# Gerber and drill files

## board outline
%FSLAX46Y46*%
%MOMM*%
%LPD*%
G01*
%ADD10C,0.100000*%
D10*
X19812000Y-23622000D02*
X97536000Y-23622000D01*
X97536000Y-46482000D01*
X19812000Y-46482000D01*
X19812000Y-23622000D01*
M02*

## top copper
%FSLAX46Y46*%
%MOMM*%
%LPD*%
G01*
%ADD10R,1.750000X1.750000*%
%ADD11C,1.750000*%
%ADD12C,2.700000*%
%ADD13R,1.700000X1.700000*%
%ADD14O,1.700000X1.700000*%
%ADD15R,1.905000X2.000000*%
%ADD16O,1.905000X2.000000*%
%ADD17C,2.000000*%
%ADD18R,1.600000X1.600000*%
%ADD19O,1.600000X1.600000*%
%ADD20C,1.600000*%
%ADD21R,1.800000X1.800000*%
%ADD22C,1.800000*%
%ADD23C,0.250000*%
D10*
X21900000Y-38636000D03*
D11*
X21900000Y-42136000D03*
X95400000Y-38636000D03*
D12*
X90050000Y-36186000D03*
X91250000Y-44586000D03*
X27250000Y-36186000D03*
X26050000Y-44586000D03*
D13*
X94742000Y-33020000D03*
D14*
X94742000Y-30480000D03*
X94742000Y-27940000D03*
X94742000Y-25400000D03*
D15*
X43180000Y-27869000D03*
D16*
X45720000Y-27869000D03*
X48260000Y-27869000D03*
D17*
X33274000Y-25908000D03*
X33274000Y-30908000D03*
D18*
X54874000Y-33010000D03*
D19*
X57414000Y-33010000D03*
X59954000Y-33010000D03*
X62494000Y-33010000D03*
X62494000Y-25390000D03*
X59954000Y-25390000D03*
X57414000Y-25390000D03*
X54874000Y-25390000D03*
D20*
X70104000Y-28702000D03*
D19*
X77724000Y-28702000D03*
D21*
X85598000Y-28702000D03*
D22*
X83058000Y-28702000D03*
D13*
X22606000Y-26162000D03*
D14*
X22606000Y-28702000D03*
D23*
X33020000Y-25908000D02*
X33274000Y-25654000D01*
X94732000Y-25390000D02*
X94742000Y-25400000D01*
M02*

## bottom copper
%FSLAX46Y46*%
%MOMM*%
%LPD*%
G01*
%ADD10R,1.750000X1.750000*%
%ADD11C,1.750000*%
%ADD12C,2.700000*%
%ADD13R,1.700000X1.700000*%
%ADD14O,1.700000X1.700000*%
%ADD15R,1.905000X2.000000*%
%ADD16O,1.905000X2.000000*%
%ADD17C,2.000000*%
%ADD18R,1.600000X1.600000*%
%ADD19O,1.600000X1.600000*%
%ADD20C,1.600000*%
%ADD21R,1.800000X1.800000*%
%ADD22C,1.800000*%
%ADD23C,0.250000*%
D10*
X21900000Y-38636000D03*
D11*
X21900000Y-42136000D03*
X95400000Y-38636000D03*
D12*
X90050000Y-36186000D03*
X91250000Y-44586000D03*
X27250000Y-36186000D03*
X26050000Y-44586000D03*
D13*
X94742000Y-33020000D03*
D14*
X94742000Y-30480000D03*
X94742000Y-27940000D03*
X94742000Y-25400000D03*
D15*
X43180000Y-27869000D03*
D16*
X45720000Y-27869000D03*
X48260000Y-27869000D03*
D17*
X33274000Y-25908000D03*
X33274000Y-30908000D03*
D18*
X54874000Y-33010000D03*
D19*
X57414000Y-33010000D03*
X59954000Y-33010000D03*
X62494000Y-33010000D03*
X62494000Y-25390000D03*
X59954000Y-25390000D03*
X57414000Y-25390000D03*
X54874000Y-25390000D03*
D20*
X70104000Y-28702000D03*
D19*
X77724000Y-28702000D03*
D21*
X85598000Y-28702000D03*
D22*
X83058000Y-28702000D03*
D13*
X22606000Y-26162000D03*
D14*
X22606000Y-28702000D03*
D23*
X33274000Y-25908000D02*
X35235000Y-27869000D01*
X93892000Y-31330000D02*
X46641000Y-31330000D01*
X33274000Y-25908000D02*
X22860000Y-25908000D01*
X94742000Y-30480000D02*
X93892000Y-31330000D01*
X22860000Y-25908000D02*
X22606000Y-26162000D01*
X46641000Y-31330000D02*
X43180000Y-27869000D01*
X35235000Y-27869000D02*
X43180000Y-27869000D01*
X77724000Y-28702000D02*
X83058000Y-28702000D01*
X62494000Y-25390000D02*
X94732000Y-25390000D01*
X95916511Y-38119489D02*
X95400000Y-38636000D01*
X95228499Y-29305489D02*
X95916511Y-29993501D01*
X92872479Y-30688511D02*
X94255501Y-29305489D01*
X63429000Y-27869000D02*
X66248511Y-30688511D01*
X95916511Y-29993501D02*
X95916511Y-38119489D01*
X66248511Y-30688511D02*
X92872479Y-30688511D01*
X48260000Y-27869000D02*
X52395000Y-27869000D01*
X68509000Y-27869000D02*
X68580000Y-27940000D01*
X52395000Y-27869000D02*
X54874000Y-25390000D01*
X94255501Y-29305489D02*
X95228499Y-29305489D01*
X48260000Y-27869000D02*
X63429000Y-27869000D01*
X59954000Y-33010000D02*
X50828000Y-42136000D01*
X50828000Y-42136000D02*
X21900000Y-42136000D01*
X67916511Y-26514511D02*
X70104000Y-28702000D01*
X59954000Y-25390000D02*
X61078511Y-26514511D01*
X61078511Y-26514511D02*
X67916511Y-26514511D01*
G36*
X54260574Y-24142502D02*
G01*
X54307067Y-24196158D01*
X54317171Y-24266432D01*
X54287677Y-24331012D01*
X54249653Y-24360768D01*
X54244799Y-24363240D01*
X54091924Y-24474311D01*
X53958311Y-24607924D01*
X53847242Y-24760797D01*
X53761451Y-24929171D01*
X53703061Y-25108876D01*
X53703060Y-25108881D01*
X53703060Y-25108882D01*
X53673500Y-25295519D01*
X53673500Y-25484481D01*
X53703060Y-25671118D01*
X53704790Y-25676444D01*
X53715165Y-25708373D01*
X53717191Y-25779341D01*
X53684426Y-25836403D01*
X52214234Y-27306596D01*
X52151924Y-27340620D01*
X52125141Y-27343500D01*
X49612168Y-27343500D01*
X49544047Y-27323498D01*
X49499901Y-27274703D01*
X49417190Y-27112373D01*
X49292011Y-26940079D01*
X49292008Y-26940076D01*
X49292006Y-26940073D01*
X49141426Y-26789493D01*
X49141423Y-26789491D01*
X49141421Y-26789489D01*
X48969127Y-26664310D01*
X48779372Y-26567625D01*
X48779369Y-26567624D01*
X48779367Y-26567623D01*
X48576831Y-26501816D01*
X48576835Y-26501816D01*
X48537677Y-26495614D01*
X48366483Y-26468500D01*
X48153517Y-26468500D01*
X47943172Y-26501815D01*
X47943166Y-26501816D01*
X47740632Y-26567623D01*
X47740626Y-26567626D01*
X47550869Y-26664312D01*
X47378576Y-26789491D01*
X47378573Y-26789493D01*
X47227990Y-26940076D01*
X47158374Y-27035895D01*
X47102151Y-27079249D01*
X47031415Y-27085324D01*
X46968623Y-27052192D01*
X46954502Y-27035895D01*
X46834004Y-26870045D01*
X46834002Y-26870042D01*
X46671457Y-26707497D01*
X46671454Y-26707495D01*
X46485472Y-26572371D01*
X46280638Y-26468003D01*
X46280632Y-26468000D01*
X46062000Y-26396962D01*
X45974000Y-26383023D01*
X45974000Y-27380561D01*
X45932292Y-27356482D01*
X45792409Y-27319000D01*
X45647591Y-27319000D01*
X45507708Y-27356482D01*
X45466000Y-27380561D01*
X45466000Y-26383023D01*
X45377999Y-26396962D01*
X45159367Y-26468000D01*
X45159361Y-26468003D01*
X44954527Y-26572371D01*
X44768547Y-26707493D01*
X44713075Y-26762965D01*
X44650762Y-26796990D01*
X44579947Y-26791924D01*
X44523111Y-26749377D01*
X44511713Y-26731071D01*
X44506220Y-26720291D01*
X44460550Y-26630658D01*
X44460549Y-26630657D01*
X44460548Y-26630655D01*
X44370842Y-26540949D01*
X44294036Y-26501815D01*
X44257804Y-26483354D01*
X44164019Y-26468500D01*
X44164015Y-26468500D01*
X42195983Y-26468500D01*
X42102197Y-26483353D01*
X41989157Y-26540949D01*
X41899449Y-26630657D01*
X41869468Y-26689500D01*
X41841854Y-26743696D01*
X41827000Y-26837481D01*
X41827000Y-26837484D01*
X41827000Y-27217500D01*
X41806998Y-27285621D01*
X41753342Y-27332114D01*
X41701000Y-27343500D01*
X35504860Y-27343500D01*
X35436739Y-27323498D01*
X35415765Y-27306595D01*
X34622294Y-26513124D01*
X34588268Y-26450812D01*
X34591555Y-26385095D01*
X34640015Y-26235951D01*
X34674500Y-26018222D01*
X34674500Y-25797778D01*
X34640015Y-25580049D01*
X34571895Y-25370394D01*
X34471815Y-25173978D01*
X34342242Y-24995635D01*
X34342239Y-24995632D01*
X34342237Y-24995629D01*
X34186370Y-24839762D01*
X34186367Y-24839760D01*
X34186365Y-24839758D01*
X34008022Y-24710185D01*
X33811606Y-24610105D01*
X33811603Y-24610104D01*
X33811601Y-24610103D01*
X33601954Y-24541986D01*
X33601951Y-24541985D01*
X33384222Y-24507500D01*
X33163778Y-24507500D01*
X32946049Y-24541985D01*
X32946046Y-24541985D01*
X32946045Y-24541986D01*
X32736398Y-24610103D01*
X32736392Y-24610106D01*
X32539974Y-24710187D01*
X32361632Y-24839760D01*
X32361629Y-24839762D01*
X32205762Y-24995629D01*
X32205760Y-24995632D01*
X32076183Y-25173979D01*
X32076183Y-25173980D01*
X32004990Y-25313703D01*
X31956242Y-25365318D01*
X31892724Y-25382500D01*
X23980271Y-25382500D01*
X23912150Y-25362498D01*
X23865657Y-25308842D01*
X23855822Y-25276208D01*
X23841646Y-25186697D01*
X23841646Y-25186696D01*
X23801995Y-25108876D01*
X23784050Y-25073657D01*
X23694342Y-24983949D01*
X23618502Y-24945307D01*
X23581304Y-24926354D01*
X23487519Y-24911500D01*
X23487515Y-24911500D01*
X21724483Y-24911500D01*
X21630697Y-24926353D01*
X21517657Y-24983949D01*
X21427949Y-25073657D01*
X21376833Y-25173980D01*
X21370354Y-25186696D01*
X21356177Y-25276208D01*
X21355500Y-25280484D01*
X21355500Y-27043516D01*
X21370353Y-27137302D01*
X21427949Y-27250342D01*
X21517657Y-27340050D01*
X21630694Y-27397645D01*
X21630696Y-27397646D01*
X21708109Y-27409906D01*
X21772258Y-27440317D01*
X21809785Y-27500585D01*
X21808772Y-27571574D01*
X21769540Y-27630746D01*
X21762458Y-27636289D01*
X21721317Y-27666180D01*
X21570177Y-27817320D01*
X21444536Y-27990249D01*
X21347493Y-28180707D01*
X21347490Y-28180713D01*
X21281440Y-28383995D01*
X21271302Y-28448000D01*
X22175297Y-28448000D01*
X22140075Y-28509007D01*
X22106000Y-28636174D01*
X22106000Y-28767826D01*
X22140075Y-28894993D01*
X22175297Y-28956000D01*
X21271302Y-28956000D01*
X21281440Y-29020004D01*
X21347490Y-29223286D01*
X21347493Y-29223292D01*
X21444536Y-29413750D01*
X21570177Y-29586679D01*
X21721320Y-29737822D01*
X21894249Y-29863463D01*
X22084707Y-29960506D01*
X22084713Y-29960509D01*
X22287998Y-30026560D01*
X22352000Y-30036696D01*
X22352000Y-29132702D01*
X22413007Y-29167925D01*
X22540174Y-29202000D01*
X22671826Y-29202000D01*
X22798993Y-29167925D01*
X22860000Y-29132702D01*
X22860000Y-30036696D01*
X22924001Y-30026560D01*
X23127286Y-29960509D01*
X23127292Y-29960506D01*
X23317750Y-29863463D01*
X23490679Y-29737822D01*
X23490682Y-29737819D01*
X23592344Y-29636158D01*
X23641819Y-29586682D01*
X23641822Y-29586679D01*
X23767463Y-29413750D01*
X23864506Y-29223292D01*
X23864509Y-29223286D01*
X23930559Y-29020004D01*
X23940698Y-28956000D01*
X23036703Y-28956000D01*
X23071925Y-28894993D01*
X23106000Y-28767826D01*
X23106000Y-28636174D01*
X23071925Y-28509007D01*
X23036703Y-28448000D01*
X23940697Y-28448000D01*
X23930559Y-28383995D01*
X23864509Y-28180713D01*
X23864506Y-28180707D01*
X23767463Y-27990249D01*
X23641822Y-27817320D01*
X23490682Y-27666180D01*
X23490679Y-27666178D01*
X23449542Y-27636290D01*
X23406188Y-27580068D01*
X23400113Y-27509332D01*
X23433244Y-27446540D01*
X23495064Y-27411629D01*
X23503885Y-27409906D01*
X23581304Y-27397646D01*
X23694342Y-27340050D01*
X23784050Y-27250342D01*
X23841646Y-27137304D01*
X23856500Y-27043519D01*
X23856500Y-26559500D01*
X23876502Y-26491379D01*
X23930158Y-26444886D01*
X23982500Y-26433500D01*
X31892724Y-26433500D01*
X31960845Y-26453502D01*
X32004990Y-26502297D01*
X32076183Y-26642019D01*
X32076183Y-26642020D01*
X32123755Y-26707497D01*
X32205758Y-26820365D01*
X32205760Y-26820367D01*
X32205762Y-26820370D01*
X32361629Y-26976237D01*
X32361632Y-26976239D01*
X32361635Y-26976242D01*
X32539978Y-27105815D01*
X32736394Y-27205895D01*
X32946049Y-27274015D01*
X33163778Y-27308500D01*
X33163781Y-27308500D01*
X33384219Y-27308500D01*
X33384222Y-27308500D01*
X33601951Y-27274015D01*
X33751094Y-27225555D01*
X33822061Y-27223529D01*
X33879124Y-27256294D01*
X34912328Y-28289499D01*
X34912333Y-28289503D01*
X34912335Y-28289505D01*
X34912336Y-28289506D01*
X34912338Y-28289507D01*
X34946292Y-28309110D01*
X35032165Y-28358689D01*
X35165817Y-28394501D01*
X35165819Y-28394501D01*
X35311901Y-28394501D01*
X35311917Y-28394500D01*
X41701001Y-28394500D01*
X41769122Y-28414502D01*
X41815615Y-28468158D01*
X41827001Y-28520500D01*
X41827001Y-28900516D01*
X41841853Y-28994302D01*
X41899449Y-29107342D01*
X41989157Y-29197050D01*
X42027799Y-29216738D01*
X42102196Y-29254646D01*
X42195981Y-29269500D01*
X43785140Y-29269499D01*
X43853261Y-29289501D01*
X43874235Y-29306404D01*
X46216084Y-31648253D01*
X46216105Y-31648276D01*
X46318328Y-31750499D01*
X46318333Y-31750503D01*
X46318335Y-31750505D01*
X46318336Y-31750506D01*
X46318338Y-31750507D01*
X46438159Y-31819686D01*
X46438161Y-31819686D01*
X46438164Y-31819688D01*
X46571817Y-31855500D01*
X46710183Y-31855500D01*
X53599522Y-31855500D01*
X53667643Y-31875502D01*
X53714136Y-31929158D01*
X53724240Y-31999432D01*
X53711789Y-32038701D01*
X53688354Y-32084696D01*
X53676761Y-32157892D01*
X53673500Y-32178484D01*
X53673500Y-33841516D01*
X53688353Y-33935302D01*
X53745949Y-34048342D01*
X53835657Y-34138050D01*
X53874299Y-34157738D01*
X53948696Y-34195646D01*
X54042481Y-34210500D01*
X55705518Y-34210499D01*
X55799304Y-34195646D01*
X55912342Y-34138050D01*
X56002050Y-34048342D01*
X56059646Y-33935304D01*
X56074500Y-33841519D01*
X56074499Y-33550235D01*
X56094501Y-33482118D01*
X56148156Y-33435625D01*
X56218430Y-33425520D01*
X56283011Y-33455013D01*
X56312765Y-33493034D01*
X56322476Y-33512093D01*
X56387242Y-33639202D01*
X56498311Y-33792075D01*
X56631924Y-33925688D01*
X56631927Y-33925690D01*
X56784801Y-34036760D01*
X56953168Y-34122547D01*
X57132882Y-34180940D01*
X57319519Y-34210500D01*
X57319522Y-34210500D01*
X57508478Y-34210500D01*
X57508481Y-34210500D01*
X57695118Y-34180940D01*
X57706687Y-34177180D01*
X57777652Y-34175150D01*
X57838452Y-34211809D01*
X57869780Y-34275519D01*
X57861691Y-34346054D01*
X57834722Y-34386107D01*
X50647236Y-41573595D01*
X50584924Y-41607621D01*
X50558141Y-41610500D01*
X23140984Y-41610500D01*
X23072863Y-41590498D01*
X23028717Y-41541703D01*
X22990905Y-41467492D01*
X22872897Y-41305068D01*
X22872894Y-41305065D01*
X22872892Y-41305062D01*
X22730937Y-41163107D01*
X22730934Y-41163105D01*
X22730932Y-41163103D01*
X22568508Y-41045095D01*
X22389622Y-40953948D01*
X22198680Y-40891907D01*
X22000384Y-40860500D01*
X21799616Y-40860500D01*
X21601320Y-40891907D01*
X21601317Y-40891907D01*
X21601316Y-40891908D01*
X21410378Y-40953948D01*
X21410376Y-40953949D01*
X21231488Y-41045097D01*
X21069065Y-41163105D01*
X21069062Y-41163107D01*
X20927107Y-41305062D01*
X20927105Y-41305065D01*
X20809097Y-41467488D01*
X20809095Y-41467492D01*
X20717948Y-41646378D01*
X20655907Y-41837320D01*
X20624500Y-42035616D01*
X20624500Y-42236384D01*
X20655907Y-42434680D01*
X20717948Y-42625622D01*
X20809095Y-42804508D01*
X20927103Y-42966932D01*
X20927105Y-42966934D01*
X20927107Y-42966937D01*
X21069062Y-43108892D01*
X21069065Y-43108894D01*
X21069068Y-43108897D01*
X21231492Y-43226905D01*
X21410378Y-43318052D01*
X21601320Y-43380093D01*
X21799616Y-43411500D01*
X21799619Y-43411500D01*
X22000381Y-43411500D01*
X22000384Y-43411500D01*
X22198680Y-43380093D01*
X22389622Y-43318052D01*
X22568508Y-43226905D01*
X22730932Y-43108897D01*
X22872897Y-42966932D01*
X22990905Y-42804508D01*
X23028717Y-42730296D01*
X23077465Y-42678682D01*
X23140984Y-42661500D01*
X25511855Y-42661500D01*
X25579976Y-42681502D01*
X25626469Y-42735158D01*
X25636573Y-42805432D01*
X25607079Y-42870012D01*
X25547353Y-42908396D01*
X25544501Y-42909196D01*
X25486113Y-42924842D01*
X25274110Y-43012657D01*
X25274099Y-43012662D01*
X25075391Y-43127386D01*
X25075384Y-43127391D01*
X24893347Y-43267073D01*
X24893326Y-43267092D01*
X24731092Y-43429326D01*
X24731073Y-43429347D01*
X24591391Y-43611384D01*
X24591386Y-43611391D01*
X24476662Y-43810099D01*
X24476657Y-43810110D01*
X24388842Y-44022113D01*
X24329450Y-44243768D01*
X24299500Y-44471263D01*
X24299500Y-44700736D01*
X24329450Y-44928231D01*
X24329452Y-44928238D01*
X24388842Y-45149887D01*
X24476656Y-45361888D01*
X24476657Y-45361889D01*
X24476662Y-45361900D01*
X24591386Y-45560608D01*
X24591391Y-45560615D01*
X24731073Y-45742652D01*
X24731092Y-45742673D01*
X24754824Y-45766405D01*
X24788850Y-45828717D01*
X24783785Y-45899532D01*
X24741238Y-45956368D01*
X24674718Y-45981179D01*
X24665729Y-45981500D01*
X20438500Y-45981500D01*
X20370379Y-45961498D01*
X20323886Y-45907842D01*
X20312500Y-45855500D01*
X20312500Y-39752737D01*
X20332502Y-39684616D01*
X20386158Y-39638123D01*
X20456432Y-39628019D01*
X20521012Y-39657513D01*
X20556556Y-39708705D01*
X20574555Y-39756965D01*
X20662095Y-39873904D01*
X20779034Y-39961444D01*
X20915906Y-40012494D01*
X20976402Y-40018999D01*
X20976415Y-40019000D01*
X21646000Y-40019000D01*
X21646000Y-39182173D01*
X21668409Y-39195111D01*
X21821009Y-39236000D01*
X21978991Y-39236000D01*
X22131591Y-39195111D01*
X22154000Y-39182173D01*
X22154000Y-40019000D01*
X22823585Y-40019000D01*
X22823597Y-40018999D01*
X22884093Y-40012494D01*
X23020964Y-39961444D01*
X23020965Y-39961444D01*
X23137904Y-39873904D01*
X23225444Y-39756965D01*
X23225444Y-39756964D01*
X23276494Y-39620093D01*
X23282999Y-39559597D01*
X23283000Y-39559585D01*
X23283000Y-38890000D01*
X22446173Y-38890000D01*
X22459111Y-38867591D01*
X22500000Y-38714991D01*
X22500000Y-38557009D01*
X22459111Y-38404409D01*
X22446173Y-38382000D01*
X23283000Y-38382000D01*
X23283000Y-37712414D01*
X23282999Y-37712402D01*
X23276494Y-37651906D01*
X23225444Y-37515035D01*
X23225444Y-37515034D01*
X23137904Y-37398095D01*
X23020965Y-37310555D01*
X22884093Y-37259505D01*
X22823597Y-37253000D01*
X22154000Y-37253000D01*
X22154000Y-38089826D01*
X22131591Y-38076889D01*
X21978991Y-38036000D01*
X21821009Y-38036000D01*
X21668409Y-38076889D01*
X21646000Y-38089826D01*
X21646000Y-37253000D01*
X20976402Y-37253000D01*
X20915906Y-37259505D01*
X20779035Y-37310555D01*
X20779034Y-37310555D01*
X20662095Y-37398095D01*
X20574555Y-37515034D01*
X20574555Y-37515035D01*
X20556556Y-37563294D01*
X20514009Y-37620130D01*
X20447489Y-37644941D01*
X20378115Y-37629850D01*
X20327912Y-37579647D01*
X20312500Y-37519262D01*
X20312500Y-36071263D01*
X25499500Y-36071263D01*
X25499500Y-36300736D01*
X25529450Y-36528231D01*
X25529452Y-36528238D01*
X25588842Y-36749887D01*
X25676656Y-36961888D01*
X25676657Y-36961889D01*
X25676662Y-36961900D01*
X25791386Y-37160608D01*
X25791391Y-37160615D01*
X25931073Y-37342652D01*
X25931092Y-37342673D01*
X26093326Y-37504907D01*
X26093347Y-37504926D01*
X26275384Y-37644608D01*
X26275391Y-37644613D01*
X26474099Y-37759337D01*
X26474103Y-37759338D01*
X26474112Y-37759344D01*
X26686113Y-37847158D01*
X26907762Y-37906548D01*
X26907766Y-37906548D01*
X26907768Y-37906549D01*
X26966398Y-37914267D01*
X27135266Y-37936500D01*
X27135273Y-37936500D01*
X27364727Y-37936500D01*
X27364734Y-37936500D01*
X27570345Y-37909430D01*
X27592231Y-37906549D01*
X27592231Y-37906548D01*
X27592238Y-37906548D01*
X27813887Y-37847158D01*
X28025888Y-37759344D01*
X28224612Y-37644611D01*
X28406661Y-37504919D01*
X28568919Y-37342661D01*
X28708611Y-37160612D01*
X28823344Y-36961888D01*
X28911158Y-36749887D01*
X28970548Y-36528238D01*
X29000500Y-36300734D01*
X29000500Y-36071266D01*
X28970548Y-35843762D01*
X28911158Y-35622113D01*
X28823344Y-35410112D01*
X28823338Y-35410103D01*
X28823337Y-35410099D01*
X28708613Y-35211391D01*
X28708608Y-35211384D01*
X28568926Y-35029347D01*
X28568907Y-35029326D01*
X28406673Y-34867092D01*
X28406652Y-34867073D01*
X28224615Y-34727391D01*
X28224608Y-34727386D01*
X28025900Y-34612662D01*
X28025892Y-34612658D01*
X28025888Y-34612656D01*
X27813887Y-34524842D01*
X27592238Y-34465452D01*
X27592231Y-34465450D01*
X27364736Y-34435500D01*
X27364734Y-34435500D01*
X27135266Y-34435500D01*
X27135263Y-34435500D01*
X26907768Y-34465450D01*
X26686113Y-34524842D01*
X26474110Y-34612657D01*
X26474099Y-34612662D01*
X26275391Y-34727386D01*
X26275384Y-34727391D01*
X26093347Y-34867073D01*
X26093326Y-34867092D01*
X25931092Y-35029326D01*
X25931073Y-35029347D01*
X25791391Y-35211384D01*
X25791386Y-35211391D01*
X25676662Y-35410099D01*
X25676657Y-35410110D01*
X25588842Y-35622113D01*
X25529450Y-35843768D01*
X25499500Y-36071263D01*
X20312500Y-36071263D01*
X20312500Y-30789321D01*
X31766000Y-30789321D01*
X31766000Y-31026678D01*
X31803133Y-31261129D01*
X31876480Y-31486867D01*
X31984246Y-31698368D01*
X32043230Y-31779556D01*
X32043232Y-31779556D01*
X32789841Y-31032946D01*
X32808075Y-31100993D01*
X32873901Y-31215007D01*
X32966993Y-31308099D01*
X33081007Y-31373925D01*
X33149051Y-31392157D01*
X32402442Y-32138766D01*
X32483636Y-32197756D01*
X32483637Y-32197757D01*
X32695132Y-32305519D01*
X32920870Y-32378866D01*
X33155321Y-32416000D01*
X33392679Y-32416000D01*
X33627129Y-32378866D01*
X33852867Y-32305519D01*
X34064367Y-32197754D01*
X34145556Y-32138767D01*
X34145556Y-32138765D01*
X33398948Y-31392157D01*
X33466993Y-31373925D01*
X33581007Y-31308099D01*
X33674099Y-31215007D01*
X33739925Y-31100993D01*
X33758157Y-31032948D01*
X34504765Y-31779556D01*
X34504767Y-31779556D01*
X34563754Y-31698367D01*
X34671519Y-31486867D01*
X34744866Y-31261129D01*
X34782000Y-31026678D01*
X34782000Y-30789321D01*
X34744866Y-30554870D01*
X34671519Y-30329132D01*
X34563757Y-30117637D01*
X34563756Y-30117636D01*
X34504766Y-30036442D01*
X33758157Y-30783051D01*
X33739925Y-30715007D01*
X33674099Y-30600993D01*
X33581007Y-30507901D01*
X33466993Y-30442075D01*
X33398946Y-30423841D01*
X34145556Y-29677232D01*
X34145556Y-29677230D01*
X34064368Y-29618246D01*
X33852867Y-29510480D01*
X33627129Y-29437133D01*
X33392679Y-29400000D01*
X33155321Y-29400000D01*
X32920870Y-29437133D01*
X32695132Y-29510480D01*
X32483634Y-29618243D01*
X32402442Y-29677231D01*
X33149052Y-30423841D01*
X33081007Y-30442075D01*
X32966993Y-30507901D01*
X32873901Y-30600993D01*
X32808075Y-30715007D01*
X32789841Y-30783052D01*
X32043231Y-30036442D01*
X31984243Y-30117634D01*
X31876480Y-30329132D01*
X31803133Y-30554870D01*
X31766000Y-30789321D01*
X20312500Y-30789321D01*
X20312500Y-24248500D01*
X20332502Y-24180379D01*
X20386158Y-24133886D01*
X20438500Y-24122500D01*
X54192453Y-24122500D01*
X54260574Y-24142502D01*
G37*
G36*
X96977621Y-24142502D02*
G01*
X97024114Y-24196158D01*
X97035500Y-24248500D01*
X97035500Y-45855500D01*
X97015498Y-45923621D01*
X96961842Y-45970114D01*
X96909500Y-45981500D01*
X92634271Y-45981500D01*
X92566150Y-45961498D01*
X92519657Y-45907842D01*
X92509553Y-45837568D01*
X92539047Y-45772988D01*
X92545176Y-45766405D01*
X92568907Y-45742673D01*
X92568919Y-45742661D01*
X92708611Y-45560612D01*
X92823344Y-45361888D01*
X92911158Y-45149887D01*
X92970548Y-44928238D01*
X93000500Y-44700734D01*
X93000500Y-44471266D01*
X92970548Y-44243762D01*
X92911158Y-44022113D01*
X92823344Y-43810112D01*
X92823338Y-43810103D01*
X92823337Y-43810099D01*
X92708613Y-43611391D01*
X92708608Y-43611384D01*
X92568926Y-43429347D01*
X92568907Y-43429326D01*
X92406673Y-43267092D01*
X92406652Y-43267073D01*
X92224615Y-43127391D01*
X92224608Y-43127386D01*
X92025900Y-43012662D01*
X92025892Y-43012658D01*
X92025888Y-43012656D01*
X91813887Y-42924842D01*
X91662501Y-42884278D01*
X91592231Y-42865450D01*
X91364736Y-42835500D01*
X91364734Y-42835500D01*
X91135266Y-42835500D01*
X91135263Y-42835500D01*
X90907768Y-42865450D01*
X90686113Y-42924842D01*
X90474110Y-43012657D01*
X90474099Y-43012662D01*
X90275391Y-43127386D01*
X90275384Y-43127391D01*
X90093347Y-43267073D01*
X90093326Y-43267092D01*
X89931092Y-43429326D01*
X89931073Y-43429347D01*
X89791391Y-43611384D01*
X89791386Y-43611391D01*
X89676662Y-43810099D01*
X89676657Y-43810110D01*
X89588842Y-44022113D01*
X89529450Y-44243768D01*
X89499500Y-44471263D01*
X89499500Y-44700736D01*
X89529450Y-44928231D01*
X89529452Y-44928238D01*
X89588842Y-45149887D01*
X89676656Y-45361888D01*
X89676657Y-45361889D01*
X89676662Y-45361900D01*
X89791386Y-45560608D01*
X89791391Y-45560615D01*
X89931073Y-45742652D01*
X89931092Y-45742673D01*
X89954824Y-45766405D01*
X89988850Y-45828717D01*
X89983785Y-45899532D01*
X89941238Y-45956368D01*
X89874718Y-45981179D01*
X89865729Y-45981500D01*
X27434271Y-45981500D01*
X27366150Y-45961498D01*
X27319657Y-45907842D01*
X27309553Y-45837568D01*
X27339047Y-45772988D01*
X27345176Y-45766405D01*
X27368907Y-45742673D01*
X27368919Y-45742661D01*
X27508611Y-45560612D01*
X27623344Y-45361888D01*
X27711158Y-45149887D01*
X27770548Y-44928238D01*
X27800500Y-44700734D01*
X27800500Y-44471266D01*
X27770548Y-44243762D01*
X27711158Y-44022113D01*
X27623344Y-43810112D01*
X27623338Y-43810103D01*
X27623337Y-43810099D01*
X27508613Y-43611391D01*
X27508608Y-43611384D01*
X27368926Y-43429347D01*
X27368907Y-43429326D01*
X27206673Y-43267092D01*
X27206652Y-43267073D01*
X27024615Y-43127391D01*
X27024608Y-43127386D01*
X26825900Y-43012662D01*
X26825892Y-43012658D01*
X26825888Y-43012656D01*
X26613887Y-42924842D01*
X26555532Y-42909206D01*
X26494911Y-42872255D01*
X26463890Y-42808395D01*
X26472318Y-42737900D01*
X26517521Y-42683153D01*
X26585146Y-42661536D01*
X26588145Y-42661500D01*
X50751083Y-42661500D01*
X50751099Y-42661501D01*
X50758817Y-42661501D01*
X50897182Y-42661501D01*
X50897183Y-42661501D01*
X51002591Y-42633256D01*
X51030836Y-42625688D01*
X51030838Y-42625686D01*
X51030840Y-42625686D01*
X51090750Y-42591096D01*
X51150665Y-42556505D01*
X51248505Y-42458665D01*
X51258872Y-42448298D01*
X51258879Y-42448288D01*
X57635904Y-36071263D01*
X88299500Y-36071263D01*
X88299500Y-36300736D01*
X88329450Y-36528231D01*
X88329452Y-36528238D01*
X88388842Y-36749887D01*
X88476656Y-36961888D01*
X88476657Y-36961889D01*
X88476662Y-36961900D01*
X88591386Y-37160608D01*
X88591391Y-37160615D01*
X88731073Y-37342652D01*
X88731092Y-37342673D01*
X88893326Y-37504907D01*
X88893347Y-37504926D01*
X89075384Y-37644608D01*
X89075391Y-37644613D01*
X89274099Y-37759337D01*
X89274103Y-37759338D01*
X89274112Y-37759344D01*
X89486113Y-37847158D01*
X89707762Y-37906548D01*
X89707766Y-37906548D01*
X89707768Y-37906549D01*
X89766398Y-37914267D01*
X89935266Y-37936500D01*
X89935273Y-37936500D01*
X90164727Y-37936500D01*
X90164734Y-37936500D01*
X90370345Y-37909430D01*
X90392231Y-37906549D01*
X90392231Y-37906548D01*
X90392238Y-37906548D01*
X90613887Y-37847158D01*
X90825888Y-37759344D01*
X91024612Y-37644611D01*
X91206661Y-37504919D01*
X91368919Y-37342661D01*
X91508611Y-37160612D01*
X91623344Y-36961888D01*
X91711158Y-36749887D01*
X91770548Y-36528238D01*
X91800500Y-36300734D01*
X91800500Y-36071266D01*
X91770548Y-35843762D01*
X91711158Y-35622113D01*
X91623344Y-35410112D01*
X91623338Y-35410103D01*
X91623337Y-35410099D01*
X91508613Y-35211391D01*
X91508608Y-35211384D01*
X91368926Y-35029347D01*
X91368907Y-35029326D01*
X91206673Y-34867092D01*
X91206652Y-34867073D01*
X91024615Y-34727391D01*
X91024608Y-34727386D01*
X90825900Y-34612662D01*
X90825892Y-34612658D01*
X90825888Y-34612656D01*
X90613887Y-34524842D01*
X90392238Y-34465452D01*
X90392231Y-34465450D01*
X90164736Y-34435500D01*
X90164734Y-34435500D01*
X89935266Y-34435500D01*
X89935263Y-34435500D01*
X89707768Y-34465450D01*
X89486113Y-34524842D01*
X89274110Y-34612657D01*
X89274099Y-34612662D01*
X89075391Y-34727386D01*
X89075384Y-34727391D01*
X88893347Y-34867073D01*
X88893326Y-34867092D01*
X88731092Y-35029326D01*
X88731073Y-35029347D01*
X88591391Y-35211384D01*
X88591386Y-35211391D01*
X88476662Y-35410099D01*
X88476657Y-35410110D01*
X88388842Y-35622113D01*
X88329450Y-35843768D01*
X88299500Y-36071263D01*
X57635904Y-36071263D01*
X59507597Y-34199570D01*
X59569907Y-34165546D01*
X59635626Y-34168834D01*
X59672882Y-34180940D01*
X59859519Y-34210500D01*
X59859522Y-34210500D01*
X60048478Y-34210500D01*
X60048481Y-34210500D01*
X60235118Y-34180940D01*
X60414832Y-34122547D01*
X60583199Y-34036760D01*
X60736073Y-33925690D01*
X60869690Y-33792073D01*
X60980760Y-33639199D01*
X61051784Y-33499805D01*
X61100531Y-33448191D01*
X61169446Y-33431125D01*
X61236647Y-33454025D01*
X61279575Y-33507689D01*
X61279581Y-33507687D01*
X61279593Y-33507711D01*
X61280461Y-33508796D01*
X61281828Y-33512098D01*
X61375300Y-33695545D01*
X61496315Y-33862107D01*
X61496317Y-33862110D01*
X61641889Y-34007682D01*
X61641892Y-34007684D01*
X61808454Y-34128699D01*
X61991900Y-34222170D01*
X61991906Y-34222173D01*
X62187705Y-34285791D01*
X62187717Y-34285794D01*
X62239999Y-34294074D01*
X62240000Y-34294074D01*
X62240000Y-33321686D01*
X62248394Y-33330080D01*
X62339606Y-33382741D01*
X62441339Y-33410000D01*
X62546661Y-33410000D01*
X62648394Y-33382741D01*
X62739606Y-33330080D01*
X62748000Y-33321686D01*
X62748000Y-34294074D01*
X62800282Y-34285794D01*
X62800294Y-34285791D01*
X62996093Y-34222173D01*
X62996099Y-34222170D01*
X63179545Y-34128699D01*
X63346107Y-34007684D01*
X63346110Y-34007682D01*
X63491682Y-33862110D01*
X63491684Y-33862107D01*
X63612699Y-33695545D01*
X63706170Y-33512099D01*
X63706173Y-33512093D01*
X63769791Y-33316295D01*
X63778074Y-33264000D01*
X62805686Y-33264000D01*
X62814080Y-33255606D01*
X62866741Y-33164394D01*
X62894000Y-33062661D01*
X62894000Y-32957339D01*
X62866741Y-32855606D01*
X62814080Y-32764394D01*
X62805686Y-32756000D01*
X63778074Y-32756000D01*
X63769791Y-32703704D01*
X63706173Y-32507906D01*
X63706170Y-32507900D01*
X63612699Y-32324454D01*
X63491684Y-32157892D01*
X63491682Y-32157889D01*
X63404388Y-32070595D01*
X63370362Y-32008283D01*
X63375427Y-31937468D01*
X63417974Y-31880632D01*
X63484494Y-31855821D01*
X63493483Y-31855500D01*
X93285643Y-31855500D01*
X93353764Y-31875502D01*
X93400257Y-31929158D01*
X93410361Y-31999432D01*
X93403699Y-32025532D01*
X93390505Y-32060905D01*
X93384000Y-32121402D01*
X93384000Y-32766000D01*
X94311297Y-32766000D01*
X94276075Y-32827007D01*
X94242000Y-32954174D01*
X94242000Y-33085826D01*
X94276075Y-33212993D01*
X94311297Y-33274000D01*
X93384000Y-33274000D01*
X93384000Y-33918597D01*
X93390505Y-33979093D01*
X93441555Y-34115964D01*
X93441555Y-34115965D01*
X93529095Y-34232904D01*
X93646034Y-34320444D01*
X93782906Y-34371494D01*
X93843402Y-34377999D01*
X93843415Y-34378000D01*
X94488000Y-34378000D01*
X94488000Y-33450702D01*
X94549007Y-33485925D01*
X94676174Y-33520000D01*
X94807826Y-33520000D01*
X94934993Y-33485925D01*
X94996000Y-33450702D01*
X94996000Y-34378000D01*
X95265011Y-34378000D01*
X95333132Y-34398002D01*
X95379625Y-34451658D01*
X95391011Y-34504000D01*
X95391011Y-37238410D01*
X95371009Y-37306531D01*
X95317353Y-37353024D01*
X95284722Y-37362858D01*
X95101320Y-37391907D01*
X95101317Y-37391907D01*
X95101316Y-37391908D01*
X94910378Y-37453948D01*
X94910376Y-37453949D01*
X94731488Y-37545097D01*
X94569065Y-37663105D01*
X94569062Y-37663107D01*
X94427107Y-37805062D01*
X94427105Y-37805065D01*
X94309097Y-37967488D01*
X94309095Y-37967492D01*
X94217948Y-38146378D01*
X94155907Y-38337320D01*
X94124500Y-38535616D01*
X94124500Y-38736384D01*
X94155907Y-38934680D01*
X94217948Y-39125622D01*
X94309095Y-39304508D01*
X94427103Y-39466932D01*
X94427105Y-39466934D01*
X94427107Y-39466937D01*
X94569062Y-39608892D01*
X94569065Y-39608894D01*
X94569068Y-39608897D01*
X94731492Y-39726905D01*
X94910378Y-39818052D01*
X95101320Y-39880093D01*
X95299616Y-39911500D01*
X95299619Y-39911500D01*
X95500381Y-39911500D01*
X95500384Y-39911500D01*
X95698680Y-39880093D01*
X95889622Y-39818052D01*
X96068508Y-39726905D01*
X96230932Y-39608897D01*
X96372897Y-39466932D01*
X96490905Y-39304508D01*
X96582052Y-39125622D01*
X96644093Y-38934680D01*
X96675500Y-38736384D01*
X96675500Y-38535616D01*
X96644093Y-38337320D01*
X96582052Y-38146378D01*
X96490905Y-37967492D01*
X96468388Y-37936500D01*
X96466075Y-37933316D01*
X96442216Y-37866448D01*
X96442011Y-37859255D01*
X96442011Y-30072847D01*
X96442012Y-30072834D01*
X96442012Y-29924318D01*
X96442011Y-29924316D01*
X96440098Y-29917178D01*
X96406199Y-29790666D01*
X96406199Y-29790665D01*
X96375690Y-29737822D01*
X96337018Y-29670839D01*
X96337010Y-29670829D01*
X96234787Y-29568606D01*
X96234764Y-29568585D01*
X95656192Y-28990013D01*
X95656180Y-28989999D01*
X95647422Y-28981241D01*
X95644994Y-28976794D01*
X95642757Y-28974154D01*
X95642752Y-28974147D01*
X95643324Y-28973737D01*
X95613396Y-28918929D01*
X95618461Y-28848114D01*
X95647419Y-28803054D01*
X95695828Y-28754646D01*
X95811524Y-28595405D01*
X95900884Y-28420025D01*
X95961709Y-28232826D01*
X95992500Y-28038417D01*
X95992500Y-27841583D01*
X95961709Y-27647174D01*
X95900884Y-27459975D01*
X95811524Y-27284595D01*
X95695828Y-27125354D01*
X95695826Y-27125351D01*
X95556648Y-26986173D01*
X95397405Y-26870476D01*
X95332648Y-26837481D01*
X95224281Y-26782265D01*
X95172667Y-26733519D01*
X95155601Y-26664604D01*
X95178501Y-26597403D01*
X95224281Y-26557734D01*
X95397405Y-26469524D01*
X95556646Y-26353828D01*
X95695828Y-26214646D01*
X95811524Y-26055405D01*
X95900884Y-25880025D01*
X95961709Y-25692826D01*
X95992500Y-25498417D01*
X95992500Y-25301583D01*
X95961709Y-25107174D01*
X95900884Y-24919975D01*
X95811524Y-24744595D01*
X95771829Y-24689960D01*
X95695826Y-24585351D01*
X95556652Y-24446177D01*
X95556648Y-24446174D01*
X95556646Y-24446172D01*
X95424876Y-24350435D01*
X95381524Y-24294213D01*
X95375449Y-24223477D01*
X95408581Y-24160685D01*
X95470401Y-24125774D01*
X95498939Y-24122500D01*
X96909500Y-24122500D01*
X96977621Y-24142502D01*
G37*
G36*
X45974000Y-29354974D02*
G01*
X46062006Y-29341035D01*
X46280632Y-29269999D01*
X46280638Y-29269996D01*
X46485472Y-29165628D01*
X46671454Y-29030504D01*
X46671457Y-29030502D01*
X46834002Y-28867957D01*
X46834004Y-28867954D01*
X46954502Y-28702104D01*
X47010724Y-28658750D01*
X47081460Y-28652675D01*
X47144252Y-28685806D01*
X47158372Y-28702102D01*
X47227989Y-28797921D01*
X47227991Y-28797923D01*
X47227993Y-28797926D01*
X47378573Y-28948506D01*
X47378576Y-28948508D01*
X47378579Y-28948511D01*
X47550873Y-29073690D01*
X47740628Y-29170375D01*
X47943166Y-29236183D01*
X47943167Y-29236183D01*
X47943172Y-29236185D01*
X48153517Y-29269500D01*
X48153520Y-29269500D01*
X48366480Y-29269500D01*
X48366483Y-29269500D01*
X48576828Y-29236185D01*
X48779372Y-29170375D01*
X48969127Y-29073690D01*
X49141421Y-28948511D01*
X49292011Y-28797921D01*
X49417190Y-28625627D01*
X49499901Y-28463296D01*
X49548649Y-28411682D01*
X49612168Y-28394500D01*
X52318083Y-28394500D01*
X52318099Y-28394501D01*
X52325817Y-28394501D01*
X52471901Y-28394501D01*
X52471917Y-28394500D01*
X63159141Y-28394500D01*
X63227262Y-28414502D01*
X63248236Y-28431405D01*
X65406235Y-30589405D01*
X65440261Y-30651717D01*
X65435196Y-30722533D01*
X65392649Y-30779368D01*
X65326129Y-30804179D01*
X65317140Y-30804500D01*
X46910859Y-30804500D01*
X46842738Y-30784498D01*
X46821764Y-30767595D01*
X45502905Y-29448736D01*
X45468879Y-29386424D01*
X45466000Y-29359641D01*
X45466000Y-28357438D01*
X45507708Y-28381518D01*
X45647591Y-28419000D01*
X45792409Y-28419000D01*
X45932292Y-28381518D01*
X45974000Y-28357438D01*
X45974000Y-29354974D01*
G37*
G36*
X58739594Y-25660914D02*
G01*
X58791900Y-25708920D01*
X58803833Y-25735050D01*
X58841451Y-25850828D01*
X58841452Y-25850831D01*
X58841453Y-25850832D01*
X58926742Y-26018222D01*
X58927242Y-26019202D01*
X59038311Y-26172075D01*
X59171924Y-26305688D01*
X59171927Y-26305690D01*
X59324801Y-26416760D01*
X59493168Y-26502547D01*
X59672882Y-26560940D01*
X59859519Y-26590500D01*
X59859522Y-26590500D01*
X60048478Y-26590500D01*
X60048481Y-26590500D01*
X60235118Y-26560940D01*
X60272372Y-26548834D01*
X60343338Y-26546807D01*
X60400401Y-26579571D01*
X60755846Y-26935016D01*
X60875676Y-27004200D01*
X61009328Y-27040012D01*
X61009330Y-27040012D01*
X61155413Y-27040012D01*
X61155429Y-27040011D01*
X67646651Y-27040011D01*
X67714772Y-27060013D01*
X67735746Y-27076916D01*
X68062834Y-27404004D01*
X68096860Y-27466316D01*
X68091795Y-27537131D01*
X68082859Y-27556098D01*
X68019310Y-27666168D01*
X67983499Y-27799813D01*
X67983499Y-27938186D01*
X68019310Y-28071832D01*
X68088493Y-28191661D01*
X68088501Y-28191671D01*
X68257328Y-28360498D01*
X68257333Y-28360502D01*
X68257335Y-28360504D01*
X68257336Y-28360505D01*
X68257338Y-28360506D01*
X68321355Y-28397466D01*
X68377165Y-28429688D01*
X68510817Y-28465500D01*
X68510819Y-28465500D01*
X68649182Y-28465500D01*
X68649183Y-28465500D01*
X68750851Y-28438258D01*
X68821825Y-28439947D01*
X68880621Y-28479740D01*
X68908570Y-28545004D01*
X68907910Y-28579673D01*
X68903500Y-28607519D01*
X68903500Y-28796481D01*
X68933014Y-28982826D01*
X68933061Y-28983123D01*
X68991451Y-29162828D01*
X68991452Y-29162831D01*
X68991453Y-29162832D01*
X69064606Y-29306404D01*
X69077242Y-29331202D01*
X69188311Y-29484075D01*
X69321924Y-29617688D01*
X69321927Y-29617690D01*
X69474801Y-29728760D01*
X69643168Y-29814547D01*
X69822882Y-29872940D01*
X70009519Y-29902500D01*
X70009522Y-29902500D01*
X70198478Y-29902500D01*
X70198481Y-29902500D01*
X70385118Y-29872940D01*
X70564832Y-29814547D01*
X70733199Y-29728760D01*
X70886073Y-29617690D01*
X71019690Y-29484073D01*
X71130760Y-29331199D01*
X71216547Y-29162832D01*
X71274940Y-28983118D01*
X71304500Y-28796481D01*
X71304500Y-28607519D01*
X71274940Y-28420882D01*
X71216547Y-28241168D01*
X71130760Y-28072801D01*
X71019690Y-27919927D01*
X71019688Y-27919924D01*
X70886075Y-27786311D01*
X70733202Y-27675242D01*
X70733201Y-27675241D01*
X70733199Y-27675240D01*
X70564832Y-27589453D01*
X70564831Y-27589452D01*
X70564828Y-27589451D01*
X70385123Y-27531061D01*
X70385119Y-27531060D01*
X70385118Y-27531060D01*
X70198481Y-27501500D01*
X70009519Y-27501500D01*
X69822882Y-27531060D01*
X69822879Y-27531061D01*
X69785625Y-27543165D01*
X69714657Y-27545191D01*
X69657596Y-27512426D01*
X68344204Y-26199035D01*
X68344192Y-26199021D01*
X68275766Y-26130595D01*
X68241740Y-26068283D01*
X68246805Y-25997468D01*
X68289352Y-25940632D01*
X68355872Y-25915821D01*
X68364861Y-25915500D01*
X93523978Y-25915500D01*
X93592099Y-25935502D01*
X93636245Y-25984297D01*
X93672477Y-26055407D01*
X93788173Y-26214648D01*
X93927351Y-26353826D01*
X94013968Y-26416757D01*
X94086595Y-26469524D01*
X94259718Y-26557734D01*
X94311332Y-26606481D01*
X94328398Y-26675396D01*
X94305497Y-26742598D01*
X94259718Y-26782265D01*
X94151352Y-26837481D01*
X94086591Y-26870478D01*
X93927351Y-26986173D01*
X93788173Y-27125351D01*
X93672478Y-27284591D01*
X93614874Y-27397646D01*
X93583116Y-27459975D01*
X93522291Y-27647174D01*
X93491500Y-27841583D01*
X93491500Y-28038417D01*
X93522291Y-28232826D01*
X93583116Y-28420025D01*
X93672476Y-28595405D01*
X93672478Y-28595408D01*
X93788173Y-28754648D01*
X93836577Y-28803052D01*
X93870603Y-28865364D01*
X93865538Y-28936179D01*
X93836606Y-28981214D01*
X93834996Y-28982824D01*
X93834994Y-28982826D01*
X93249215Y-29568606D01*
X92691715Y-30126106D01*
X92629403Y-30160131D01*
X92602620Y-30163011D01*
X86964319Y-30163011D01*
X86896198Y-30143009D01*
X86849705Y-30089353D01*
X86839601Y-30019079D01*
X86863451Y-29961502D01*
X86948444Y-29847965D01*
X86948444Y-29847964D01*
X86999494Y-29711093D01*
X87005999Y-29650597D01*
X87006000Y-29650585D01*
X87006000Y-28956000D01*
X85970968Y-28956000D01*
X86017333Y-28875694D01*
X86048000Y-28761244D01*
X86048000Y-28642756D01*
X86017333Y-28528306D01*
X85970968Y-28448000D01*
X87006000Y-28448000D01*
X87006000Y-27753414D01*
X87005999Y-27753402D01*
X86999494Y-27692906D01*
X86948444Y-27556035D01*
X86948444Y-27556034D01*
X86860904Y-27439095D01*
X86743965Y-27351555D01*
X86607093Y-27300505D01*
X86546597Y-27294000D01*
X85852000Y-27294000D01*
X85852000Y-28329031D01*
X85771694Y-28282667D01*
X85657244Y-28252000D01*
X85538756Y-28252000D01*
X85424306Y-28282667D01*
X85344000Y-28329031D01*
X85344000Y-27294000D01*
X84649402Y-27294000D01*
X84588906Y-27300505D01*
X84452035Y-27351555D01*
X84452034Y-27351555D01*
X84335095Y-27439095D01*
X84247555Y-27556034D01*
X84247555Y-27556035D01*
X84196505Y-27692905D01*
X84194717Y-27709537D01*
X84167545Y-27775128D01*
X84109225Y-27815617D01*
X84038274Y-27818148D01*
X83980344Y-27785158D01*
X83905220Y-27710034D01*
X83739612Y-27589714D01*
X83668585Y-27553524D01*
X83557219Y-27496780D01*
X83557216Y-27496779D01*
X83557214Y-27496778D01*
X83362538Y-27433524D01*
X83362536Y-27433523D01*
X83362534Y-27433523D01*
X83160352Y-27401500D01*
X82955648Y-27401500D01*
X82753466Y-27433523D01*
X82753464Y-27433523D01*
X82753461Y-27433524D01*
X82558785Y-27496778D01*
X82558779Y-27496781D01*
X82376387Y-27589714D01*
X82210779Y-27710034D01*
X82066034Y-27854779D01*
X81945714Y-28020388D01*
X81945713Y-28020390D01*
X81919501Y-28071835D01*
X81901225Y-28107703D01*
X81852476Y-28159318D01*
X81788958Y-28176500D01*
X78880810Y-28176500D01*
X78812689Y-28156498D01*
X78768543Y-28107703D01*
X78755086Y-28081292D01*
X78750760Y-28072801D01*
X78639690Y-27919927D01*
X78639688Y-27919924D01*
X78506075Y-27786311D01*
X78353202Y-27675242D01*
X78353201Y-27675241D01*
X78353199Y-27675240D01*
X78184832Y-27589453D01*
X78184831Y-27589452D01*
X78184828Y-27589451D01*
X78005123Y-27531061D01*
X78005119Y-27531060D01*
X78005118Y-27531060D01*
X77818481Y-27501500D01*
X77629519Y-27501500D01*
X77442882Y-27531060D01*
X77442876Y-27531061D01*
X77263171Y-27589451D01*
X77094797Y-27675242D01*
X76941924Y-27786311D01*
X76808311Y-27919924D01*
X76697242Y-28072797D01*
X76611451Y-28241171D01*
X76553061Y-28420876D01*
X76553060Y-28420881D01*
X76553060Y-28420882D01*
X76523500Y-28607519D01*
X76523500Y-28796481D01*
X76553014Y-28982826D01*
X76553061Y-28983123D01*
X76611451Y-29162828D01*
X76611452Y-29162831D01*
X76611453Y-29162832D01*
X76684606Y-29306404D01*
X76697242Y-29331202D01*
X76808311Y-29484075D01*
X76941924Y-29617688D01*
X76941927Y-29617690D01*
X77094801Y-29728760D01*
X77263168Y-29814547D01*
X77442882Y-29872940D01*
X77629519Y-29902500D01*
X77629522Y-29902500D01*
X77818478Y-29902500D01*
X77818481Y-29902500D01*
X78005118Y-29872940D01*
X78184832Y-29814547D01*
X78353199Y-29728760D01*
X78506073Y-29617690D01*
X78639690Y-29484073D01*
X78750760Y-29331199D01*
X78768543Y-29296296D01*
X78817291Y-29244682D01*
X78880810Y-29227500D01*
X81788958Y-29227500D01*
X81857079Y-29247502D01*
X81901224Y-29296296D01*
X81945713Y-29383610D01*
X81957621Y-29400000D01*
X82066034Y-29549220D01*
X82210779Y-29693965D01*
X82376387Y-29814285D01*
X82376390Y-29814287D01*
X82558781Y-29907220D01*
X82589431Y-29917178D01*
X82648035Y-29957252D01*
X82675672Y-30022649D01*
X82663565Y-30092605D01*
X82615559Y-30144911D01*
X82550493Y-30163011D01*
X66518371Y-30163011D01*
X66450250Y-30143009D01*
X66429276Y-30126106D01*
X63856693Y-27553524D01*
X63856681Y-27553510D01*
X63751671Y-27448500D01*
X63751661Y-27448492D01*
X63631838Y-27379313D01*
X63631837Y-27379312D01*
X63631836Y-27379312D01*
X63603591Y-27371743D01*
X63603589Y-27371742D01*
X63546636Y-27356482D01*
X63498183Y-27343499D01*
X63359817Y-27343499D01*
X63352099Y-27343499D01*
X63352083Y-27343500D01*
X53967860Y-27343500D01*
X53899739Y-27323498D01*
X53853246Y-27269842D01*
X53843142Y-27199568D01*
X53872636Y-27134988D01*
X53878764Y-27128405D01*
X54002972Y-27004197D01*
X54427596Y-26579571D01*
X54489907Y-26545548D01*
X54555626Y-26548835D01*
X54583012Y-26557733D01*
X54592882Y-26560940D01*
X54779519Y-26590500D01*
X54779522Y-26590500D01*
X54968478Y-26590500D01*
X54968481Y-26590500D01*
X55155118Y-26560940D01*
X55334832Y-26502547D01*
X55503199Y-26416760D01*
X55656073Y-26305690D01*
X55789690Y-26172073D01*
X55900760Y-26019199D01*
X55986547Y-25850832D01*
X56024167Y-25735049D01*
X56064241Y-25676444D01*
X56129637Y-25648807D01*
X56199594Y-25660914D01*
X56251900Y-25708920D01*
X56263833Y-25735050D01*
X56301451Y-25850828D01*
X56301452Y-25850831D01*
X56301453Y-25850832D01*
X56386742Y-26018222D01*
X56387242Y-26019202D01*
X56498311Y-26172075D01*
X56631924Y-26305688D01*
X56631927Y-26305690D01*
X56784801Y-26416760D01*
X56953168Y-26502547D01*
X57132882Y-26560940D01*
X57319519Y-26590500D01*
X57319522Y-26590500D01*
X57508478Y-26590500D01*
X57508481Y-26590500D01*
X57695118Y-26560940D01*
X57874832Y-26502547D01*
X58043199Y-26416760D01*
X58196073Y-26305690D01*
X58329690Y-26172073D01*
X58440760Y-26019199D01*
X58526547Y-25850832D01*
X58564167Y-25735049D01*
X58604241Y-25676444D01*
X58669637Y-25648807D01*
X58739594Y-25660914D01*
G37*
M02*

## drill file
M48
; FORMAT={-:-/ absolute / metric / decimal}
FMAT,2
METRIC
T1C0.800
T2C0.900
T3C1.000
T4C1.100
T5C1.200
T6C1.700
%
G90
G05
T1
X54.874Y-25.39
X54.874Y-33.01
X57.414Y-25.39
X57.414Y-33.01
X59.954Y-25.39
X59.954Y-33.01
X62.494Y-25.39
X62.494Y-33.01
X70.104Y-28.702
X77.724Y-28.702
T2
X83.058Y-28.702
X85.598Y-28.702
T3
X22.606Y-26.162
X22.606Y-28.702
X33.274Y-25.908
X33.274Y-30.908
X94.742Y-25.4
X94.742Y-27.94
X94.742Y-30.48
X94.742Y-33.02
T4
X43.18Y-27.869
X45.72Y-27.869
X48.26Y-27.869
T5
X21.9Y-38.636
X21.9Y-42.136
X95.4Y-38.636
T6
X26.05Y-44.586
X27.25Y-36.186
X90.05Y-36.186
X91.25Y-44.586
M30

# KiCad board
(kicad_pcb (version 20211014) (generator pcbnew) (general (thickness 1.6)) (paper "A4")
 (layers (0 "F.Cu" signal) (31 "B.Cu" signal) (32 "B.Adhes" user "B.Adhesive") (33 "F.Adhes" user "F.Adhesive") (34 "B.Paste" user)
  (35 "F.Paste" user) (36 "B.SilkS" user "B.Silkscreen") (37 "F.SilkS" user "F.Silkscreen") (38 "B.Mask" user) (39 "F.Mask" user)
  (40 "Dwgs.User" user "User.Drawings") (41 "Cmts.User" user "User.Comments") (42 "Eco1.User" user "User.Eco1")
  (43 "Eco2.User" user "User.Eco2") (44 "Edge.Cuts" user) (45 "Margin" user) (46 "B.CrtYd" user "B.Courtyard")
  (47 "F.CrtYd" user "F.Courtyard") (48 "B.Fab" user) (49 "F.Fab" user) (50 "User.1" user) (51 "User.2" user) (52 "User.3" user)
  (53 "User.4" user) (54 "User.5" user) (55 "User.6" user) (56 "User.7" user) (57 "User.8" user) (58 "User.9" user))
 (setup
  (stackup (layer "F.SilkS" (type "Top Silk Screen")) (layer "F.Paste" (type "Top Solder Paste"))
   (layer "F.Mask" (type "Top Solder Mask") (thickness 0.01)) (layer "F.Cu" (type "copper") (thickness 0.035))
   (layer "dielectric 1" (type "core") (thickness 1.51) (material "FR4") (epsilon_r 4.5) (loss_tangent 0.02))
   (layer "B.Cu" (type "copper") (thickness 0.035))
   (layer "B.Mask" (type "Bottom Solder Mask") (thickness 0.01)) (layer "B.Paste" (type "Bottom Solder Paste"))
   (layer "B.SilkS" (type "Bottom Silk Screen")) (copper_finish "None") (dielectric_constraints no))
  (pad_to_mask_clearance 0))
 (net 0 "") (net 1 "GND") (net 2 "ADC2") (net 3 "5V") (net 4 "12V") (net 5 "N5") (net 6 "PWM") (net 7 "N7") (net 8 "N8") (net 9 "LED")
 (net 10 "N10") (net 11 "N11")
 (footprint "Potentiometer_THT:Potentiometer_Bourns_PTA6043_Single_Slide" (layer "F.Cu") (at 21.9 38.636)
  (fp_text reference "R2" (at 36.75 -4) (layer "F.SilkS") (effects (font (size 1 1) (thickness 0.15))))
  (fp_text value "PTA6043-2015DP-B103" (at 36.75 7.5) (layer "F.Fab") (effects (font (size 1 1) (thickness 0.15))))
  (pad "1" thru_hole rect (at 0 0) (size 1.75 1.75) (drill 1.2) (layers *.Cu *.Mask) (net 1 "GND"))
  (pad "2" thru_hole circle (at 0 3.5) (size 1.75 1.75) (drill 1.2) (layers *.Cu *.Mask) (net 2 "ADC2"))
  (pad "3" thru_hole circle (at 73.5 0) (size 1.75 1.75) (drill 1.2) (layers *.Cu *.Mask) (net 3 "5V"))
  (pad "MP" thru_hole circle (at 68.15 -2.45) (size 2.7 2.7) (drill 1.7) (layers *.Cu *.Mask))
  (pad "MP" thru_hole circle (at 69.35 5.95) (size 2.7 2.7) (drill 1.7) (layers *.Cu *.Mask))
  (pad "MP" thru_hole circle (at 5.35 -2.45) (size 2.7 2.7) (drill 1.7) (layers *.Cu *.Mask))
  (pad "MP" thru_hole circle (at 4.15 5.95) (size 2.7 2.7) (drill 1.7) (layers *.Cu *.Mask)))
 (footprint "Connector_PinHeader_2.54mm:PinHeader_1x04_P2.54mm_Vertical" (layer "F.Cu") (at 94.742 33.02 180)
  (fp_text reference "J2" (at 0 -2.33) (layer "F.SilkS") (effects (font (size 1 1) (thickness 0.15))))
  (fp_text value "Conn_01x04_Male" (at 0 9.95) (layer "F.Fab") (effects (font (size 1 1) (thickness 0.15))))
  (pad "1" thru_hole rect (at 0 0 180) (size 1.7 1.7) (drill 1) (layers *.Cu *.Mask) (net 1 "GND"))
  (pad "2" thru_hole oval (at 0 2.54 180) (size 1.7 1.7) (drill 1) (layers *.Cu *.Mask) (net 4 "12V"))
  (pad "3" thru_hole oval (at 0 5.08 180) (size 1.7 1.7) (drill 1) (layers *.Cu *.Mask) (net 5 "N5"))
  (pad "4" thru_hole oval (at 0 7.62 180) (size 1.7 1.7) (drill 1) (layers *.Cu *.Mask) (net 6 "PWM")))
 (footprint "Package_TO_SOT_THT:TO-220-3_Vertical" (layer "F.Cu") (at 43.18 27.869)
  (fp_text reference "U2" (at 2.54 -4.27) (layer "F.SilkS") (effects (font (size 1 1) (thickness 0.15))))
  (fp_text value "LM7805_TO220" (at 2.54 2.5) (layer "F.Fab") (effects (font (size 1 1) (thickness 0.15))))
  (pad "1" thru_hole rect (at 0 0) (size 1.905 2) (drill 1.1) (layers *.Cu *.Mask) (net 4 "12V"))
  (pad "2" thru_hole oval (at 2.54 0) (size 1.905 2) (drill 1.1) (layers *.Cu *.Mask) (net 1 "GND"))
  (pad "3" thru_hole oval (at 5.08 0) (size 1.905 2) (drill 1.1) (layers *.Cu *.Mask) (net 3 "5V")))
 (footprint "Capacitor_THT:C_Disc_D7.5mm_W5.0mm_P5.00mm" (layer "F.Cu") (at 33.274 25.908 -90)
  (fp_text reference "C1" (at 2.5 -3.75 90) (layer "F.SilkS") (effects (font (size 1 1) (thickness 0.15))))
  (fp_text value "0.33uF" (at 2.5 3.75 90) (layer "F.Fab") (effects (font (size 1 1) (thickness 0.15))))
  (pad "1" thru_hole circle (at 0 0 270) (size 2 2) (drill 1) (layers *.Cu *.Mask) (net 4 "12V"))
  (pad "2" thru_hole circle (at 5 0 270) (size 2 2) (drill 1) (layers *.Cu *.Mask) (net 1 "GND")))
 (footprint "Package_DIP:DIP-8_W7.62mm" (layer "F.Cu") (at 54.874 33.01 90)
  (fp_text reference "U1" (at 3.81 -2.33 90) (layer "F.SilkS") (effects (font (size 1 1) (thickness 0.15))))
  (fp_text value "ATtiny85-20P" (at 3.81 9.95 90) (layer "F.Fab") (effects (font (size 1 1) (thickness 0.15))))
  (pad "1" thru_hole rect (at 0 0 90) (size 1.6 1.6) (drill 0.8) (layers *.Cu *.Mask) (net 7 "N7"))
  (pad "2" thru_hole oval (at 0 2.54 90) (size 1.6 1.6) (drill 0.8) (layers *.Cu *.Mask) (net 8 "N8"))
  (pad "3" thru_hole oval (at 0 5.08 90) (size 1.6 1.6) (drill 0.8) (layers *.Cu *.Mask) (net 2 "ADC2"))
  (pad "4" thru_hole oval (at 0 7.62 90) (size 1.6 1.6) (drill 0.8) (layers *.Cu *.Mask) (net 1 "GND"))
  (pad "5" thru_hole oval (at 7.62 7.62 90) (size 1.6 1.6) (drill 0.8) (layers *.Cu *.Mask) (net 6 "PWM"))
  (pad "6" thru_hole oval (at 7.62 5.08 90) (size 1.6 1.6) (drill 0.8) (layers *.Cu *.Mask) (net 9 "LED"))
  (pad "7" thru_hole oval (at 7.62 2.54 90) (size 1.6 1.6) (drill 0.8) (layers *.Cu *.Mask) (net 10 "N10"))
  (pad "8" thru_hole oval (at 7.62 0 90) (size 1.6 1.6) (drill 0.8) (layers *.Cu *.Mask) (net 3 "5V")))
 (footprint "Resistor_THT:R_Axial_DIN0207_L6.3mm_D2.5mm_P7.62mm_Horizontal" (layer "F.Cu") (at 70.104 28.702)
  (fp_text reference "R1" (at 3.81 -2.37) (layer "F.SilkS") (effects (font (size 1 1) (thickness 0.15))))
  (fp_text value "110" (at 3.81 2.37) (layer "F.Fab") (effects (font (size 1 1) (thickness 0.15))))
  (pad "1" thru_hole circle (at 0 0) (size 1.6 1.6) (drill 0.8) (layers *.Cu *.Mask) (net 9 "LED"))
  (pad "2" thru_hole oval (at 7.62 0) (size 1.6 1.6) (drill 0.8) (layers *.Cu *.Mask) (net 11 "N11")))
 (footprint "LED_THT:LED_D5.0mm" (layer "F.Cu") (at 85.598 28.702 180)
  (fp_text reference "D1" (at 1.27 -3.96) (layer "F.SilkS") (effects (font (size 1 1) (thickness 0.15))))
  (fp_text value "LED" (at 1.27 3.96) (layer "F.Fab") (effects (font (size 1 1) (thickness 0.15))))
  (pad "1" thru_hole rect (at 0 0 180) (size 1.8 1.8) (drill 0.9) (layers *.Cu *.Mask) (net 1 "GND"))
  (pad "2" thru_hole circle (at 2.54 0 180) (size 1.8 1.8) (drill 0.9) (layers *.Cu *.Mask) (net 11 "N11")))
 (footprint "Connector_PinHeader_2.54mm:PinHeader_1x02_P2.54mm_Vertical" (layer "F.Cu") (at 22.606 26.162)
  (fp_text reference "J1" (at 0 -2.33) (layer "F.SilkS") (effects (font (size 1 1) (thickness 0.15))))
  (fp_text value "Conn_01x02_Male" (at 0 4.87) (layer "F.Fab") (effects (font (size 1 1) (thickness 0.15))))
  (pad "1" thru_hole rect (at 0 0) (size 1.7 1.7) (drill 1) (layers *.Cu *.Mask) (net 4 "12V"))
  (pad "2" thru_hole oval (at 0 2.54) (size 1.7 1.7) (drill 1) (layers *.Cu *.Mask) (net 1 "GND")))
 (gr_rect (start 19.812 23.622) (end 97.536 46.482) (layer "Edge.Cuts") (width 0.1) (fill none))
 (segment (start 33.02 25.908) (end 33.274 25.654) (width 0.25) (layer "F.Cu") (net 4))
 (segment (start 33.274 25.908) (end 35.235 27.869) (width 0.25) (layer "B.Cu") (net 4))
 (segment (start 93.892 31.33) (end 46.641 31.33) (width 0.25) (layer "B.Cu") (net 4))
 (segment (start 33.274 25.908) (end 22.86 25.908) (width 0.25) (layer "B.Cu") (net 4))
 (segment (start 94.742 30.48) (end 93.892 31.33) (width 0.25) (layer "B.Cu") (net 4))
 (segment (start 22.86 25.908) (end 22.606 26.162) (width 0.25) (layer "B.Cu") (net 4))
 (segment (start 46.641 31.33) (end 43.18 27.869) (width 0.25) (layer "B.Cu") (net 4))
 (segment (start 35.235 27.869) (end 43.18 27.869) (width 0.25) (layer "B.Cu") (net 4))
 (segment (start 77.724 28.702) (end 83.058 28.702) (width 0.25) (layer "B.Cu") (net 11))
 (segment (start 94.732 25.39) (end 94.742 25.4) (width 0.25) (layer "F.Cu") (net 6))
 (segment (start 62.494 25.39) (end 94.732 25.39) (width 0.25) (layer "B.Cu") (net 6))
 (segment (start 95.916511 38.119489) (end 95.4 38.636) (width 0.25) (layer "B.Cu") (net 3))
 (segment (start 95.228499 29.305489) (end 95.916511 29.993501) (width 0.25) (layer "B.Cu") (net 3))
 (segment (start 92.872479 30.688511) (end 94.255501 29.305489) (width 0.25) (layer "B.Cu") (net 3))
 (segment (start 63.429 27.869) (end 66.248511 30.688511) (width 0.25) (layer "B.Cu") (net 3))
 (segment (start 95.916511 29.993501) (end 95.916511 38.119489) (width 0.25) (layer "B.Cu") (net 3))
 (segment (start 66.248511 30.688511) (end 92.872479 30.688511) (width 0.25) (layer "B.Cu") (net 3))
 (segment (start 48.26 27.869) (end 52.395 27.869) (width 0.25) (layer "B.Cu") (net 3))
 (segment (start 68.509 27.869) (end 68.58 27.94) (width 0.25) (layer "B.Cu") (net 3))
 (segment (start 52.395 27.869) (end 54.874 25.39) (width 0.25) (layer "B.Cu") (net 3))
 (segment (start 94.255501 29.305489) (end 95.228499 29.305489) (width 0.25) (layer "B.Cu") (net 3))
 (segment (start 48.26 27.869) (end 63.429 27.869) (width 0.25) (layer "B.Cu") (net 3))
 (segment (start 59.954 33.01) (end 50.828 42.136) (width 0.25) (layer "B.Cu") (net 2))
 (segment (start 50.828 42.136) (end 21.9 42.136) (width 0.25) (layer "B.Cu") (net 2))
 (segment (start 67.916511 26.514511) (end 70.104 28.702) (width 0.25) (layer "B.Cu") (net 9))
 (segment (start 59.954 25.39) (end 61.078511 26.514511) (width 0.25) (layer "B.Cu") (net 9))
 (segment (start 61.078511 26.514511) (end 67.916511 26.514511) (width 0.25) (layer "B.Cu") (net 9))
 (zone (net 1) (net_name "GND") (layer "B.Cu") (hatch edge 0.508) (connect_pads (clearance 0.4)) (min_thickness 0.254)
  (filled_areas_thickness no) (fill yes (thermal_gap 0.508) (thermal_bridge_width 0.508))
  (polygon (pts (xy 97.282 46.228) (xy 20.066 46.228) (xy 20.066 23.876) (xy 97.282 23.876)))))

